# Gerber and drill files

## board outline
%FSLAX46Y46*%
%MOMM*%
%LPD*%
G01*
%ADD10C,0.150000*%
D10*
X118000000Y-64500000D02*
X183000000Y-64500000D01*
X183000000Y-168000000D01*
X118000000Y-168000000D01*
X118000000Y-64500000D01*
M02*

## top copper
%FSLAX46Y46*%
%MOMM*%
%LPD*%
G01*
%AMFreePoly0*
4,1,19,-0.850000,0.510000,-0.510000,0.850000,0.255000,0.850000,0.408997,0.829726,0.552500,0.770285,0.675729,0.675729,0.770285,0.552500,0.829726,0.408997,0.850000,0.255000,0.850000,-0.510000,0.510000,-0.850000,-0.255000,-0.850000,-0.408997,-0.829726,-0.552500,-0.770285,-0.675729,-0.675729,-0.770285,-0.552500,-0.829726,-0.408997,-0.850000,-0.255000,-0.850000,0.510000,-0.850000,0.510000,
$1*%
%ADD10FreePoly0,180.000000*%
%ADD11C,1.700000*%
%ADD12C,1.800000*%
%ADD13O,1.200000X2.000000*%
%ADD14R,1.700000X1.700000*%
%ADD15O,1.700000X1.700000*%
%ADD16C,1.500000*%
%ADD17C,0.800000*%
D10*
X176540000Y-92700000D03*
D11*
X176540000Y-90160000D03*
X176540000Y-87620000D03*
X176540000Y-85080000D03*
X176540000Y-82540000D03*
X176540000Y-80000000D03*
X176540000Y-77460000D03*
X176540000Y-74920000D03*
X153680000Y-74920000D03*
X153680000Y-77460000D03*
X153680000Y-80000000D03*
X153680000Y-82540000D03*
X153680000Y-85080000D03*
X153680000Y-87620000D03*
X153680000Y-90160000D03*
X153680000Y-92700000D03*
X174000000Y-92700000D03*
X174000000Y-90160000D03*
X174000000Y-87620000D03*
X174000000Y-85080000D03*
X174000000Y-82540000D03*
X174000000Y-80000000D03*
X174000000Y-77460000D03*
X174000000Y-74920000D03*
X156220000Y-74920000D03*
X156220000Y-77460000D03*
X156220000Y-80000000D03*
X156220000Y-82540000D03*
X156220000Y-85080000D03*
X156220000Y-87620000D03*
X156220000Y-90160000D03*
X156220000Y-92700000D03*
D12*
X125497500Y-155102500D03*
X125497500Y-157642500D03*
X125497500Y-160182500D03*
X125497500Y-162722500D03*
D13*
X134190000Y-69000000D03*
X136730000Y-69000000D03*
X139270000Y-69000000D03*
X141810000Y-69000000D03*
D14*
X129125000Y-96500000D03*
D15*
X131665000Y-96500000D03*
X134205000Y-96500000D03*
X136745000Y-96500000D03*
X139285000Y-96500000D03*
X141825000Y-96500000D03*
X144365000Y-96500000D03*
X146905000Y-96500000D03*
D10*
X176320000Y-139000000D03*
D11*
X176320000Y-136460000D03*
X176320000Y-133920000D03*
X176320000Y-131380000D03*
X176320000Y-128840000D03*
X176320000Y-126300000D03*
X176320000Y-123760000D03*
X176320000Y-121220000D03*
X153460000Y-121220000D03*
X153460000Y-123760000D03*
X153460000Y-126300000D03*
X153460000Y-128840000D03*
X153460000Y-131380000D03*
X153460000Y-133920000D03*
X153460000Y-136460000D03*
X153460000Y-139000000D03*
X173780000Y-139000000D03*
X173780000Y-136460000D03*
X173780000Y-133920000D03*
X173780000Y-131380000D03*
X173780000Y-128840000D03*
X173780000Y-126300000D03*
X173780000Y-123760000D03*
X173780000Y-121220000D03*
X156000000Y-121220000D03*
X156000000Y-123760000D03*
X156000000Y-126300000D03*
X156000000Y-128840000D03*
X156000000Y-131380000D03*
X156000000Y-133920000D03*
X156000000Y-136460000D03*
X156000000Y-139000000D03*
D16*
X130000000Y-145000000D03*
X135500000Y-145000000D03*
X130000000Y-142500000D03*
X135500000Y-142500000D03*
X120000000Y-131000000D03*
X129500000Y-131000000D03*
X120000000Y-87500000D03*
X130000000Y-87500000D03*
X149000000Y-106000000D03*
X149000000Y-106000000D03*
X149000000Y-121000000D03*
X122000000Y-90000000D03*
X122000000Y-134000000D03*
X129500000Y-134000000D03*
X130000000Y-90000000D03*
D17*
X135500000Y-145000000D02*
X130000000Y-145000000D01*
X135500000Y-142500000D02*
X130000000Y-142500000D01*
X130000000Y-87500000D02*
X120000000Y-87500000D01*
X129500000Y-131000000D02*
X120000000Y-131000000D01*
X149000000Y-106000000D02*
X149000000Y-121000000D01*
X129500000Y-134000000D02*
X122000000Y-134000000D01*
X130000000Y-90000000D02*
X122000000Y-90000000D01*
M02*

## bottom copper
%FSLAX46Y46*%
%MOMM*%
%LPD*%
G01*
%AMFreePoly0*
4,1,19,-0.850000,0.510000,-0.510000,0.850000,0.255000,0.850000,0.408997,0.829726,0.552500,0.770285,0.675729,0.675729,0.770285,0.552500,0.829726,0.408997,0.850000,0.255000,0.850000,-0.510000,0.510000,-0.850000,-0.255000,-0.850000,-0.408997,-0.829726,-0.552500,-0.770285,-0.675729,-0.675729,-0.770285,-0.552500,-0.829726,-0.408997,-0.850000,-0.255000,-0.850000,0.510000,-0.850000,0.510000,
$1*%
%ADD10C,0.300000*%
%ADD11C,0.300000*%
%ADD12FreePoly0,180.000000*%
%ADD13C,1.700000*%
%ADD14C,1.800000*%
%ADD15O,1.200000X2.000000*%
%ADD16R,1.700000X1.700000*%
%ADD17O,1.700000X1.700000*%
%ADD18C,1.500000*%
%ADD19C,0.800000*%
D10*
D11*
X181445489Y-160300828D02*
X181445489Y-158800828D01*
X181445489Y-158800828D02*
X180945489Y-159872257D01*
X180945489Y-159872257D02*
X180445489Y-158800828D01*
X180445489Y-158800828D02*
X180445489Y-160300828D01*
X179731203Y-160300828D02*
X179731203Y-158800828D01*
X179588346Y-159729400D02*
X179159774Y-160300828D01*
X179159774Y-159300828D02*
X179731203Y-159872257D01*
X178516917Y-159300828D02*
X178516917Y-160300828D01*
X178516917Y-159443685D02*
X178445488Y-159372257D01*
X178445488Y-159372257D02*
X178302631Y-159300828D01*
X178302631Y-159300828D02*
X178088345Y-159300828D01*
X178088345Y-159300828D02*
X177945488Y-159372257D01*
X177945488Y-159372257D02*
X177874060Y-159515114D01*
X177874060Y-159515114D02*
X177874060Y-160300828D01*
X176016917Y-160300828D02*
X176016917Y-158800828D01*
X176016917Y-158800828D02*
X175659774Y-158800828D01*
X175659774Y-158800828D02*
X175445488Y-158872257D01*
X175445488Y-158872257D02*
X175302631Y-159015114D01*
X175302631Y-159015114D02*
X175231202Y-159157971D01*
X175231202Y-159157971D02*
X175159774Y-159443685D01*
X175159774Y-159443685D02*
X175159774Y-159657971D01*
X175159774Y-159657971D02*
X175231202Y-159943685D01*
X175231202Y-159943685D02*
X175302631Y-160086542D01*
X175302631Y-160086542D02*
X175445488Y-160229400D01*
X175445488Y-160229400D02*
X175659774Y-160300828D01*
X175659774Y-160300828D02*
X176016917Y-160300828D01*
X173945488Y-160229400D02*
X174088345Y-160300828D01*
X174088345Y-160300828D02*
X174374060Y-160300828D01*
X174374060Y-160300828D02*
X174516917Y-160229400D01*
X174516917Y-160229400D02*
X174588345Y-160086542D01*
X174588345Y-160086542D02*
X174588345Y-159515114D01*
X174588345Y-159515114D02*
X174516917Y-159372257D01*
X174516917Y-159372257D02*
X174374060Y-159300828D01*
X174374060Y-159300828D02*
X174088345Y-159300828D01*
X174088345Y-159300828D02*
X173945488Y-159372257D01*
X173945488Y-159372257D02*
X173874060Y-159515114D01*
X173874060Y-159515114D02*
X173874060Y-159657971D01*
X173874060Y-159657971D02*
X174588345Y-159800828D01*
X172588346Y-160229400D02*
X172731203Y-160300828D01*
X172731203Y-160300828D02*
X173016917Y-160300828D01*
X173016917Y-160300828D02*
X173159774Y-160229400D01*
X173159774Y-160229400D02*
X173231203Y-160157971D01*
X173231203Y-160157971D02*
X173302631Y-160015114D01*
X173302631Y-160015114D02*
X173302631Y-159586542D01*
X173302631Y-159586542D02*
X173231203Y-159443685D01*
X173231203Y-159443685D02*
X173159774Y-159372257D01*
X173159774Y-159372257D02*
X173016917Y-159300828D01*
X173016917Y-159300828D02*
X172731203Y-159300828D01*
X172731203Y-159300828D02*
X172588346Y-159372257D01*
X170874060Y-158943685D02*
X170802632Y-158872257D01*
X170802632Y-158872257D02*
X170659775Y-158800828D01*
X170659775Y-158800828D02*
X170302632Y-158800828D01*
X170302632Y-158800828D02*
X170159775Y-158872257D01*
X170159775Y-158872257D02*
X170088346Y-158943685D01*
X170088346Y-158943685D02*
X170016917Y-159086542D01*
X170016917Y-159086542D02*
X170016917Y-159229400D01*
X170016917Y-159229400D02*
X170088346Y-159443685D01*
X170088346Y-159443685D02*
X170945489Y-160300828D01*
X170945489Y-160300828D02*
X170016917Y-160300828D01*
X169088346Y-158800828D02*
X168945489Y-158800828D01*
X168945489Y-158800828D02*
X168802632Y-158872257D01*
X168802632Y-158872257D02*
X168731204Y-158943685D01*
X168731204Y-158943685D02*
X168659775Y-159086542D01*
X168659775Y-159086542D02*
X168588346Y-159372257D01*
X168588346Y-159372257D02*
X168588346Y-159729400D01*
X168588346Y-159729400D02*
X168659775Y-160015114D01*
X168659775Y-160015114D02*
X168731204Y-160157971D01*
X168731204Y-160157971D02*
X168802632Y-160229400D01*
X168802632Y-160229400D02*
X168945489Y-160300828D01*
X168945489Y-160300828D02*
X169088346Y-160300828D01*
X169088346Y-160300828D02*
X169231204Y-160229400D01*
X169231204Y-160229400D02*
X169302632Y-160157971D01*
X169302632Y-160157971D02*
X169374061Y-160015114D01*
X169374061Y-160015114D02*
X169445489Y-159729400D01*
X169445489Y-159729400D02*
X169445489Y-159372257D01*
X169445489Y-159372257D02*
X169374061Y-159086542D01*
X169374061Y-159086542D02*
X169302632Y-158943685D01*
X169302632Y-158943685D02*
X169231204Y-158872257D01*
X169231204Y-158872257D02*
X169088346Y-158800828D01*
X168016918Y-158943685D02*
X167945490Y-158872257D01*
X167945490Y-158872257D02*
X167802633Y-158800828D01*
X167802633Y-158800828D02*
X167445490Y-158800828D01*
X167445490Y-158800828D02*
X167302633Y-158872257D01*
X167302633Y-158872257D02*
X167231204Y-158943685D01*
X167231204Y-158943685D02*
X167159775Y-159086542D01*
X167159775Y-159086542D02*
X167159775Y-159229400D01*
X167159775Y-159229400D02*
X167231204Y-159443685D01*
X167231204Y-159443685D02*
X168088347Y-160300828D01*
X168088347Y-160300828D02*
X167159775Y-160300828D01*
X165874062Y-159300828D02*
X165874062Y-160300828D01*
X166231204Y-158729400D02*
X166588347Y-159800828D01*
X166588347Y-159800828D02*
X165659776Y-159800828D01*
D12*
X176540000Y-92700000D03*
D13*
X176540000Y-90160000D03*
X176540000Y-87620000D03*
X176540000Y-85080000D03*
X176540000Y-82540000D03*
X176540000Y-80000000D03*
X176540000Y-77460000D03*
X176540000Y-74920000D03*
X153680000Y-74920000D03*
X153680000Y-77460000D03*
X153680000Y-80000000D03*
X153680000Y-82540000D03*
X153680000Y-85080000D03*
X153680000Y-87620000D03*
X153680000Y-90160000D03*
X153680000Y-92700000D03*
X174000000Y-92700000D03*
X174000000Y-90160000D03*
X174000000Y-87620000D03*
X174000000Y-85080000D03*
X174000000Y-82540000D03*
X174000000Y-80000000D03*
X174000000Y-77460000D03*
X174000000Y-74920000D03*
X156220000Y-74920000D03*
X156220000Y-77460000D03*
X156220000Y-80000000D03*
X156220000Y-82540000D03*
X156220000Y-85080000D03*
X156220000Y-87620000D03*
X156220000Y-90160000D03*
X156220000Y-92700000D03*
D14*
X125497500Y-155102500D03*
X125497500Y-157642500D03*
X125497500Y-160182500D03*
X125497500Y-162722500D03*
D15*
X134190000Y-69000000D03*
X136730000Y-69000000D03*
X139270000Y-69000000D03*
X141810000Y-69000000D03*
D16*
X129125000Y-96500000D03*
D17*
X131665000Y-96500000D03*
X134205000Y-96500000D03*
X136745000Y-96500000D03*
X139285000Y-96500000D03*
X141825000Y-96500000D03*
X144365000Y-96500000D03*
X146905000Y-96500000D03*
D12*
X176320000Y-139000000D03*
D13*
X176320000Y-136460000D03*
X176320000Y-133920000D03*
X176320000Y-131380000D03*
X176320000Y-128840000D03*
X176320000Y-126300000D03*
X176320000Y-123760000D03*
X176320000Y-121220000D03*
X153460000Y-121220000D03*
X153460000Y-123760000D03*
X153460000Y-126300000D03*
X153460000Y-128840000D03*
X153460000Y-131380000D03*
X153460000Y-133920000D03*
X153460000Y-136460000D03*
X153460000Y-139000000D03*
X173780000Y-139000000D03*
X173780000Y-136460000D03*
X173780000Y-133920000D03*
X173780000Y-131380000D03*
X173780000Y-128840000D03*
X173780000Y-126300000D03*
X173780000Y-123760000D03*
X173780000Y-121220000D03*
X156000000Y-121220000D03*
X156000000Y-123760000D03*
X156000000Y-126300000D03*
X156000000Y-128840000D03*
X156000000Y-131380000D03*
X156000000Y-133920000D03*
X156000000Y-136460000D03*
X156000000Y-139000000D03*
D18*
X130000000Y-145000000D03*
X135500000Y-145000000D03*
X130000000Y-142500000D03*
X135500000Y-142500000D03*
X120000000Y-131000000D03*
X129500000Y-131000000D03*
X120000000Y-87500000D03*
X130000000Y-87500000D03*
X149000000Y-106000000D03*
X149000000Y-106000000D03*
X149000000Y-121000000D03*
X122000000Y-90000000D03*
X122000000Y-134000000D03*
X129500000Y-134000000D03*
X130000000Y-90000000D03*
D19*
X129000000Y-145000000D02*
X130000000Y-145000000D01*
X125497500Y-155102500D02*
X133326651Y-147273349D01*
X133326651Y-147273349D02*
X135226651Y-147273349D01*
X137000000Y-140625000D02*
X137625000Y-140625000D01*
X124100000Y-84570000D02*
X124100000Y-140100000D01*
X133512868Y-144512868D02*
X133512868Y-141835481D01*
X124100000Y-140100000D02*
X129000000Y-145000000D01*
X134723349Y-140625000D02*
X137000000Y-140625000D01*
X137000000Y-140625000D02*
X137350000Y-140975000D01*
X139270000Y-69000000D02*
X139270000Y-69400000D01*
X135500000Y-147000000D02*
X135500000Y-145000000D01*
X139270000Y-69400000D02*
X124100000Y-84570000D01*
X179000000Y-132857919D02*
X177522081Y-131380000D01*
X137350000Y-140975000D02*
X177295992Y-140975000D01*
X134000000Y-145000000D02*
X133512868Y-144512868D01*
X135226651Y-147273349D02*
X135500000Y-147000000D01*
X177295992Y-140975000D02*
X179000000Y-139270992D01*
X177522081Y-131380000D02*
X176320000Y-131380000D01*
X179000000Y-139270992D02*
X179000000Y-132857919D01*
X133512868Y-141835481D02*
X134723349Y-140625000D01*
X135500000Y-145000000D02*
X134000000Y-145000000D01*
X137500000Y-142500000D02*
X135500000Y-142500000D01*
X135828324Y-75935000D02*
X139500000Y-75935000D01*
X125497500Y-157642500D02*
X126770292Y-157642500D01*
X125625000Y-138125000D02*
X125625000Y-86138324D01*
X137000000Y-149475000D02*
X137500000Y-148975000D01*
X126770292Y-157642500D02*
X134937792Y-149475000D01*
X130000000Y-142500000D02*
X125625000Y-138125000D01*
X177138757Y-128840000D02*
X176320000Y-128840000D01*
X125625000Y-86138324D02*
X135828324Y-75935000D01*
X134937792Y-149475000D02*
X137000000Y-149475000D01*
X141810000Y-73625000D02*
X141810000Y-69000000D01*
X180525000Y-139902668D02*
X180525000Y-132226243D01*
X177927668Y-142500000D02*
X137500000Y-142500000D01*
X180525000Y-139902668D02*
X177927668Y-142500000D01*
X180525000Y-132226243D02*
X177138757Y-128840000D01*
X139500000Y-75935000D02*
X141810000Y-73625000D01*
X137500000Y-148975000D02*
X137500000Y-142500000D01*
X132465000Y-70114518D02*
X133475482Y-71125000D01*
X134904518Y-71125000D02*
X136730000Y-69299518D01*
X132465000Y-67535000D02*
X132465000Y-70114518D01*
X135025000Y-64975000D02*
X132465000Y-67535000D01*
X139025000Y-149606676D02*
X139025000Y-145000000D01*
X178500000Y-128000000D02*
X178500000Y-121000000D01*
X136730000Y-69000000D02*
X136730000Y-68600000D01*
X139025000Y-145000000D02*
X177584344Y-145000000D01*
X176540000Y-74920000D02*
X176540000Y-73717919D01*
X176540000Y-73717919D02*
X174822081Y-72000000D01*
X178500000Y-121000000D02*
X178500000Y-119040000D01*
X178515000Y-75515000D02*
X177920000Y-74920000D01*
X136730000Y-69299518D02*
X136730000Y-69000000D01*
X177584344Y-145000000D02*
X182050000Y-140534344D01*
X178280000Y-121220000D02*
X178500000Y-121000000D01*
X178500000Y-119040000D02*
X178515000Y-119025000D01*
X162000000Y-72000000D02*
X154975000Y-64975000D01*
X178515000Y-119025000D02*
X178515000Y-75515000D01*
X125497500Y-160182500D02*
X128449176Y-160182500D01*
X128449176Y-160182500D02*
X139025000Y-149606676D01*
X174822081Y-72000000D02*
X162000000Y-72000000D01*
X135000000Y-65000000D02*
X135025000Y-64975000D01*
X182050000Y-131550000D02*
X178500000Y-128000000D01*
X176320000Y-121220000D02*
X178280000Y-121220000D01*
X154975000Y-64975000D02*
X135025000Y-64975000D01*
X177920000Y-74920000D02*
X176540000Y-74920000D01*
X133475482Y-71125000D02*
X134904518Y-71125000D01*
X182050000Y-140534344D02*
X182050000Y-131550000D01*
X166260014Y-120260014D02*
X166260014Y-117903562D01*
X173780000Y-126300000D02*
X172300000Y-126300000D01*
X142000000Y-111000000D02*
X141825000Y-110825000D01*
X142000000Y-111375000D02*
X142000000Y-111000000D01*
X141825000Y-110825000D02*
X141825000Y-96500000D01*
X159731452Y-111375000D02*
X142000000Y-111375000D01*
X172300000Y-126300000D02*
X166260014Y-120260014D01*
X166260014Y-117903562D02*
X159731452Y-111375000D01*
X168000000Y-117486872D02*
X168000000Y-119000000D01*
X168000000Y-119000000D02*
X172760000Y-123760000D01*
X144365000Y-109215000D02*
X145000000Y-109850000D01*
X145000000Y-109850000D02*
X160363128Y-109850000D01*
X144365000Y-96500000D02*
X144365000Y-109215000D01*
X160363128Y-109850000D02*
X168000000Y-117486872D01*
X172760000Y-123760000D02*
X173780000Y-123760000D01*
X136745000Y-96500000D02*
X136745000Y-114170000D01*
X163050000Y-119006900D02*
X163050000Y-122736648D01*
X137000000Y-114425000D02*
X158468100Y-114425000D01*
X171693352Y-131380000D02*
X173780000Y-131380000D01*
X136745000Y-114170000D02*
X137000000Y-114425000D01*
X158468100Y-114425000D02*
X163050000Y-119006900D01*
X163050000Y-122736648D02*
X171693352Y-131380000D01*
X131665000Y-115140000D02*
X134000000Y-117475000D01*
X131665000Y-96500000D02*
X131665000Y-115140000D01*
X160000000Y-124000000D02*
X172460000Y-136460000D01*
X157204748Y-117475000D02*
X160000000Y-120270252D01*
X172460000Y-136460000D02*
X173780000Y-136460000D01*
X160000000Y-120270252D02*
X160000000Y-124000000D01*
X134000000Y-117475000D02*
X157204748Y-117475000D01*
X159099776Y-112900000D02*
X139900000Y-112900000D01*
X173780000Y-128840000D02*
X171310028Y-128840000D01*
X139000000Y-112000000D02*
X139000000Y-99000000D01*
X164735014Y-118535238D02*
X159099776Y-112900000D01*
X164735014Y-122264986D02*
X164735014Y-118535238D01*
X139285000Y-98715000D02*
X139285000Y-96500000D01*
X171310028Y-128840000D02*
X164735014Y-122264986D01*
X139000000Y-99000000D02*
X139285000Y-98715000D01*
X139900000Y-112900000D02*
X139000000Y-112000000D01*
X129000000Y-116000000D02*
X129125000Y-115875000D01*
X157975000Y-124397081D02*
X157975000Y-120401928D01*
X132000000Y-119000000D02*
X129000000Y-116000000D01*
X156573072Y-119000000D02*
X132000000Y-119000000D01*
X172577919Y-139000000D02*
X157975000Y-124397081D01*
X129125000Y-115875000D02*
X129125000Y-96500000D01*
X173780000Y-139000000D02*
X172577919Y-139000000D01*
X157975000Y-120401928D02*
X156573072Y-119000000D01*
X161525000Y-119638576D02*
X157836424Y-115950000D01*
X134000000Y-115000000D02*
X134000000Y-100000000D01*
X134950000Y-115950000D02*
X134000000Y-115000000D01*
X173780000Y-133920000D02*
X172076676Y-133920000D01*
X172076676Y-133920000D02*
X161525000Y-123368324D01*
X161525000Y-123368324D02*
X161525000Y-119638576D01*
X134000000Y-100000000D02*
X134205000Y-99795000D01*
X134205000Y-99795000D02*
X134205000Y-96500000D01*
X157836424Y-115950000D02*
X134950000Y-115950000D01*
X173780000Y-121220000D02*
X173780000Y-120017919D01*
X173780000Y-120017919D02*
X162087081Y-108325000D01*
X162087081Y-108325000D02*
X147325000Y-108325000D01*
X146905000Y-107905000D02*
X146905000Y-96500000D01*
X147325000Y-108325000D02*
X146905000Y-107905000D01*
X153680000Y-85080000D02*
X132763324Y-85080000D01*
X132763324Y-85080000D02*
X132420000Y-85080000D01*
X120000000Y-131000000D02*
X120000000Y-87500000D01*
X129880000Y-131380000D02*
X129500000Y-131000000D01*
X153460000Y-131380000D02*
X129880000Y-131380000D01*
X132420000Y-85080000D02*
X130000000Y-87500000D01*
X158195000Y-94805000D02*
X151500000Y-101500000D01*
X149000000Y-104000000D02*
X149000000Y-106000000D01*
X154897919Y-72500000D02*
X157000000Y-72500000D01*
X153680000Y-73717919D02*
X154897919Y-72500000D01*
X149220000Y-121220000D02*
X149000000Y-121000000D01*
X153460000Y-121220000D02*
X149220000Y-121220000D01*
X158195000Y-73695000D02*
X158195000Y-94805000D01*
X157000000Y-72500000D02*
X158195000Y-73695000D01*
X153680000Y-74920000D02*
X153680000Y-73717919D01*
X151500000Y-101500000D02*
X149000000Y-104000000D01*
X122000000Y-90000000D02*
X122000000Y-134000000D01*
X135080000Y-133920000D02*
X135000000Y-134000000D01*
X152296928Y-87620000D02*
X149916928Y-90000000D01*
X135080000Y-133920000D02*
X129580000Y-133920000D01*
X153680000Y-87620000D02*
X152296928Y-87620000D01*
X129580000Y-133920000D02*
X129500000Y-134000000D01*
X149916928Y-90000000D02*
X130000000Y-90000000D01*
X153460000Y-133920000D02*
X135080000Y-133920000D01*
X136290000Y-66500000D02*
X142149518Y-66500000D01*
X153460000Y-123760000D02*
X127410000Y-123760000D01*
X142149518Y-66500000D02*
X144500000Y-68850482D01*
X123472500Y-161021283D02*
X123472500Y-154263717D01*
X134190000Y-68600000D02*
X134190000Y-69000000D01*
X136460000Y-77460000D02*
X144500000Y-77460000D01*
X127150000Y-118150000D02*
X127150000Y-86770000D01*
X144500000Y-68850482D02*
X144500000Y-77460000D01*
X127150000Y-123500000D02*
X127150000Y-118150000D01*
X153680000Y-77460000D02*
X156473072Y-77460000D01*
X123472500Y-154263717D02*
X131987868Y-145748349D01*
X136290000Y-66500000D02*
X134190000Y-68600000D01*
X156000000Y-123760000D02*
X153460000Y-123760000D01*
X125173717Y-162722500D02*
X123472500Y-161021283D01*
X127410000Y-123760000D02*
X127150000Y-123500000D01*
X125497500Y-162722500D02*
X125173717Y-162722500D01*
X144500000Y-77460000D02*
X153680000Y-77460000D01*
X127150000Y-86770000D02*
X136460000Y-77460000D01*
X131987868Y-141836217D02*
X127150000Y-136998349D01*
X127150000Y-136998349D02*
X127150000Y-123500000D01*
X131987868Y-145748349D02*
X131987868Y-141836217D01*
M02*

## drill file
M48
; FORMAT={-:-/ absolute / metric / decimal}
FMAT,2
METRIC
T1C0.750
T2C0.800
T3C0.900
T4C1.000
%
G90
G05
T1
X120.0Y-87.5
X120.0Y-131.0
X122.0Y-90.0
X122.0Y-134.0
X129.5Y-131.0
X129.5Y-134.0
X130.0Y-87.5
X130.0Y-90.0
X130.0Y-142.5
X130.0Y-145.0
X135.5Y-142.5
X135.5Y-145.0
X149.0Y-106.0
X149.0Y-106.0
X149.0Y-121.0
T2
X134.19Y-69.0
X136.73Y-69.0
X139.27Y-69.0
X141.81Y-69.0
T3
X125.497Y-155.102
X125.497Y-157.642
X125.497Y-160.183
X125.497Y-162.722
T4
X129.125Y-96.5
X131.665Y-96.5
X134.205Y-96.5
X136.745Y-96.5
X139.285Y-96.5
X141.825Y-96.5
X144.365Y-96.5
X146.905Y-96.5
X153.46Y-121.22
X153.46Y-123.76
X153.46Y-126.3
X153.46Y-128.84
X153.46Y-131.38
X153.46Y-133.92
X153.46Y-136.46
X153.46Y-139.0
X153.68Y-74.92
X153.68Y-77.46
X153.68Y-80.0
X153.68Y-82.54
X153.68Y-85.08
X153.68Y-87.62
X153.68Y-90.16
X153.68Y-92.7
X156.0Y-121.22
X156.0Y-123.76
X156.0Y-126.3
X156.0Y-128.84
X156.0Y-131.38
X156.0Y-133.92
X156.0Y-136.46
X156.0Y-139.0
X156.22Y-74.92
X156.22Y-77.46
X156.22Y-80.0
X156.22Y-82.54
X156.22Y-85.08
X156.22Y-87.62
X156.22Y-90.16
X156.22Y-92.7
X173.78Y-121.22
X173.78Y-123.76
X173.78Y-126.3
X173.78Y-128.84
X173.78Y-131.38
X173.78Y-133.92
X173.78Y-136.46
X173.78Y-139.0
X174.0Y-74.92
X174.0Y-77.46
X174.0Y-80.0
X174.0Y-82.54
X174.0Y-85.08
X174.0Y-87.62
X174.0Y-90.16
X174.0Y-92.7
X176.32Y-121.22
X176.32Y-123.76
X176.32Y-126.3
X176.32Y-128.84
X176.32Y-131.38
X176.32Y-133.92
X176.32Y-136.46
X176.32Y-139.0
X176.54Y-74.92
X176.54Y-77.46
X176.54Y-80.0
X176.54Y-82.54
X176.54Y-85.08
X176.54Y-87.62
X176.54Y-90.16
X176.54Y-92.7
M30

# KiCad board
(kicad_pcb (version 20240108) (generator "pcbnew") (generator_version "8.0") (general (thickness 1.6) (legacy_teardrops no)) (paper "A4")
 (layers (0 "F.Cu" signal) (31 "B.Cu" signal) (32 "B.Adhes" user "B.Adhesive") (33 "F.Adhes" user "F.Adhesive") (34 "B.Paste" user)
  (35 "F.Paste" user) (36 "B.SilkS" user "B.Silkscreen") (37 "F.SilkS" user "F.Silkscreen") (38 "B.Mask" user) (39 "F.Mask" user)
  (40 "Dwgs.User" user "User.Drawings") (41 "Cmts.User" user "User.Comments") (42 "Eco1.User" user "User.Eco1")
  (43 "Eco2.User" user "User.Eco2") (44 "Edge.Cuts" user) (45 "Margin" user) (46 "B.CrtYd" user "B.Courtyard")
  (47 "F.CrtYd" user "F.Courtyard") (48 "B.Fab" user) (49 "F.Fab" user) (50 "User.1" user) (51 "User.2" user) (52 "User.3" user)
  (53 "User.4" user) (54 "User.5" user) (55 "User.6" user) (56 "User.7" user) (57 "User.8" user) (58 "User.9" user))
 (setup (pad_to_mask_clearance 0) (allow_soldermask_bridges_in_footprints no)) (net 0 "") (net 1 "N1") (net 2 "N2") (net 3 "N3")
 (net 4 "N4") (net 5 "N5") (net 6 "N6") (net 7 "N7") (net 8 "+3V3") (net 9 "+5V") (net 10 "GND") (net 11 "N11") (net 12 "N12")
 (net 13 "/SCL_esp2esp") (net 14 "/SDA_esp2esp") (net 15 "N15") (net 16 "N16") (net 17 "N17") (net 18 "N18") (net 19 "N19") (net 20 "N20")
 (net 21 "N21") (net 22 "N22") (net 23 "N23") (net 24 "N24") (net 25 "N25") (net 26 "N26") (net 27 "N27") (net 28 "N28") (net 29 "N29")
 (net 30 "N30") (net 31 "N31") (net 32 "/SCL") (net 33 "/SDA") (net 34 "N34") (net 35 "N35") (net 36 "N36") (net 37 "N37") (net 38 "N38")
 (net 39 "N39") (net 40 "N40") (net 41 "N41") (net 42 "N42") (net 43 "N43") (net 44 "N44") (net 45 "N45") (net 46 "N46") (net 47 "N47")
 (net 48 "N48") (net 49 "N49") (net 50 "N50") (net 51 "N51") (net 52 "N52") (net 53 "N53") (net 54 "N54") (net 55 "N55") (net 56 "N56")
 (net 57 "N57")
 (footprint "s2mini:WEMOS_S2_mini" (layer "F.Cu") (at 176.54 92.7 180)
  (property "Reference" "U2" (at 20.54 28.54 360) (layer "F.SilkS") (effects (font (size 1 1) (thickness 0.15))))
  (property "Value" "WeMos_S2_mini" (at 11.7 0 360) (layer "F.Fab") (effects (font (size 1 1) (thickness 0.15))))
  (pad "1" thru_hole roundrect (at 0 0 180) (size 1.7 1.7) (drill 1) (layers "*.Cu" "*.Mask") (remove_unused_layers no)
   (roundrect_rratio 0.35) (chamfer_ratio 0.2) (chamfer top_left bottom_right) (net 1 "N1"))
  (pad "2" thru_hole circle (at 0 2.54 180) (size 1.7 1.7) (drill 1) (layers "*.Cu" "*.Mask") (remove_unused_layers no) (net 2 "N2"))
  (pad "3" thru_hole circle (at 0 5.08 180) (size 1.7 1.7) (drill 1) (layers "*.Cu" "*.Mask") (remove_unused_layers no) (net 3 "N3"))
  (pad "4" thru_hole circle (at 0 7.62 180) (size 1.7 1.7) (drill 1) (layers "*.Cu" "*.Mask") (remove_unused_layers no) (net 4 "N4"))
  (pad "5" thru_hole circle (at 0 10.16 180) (size 1.7 1.7) (drill 1) (layers "*.Cu" "*.Mask") (remove_unused_layers no) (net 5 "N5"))
  (pad "6" thru_hole circle (at 0 12.7 180) (size 1.7 1.7) (drill 1) (layers "*.Cu" "*.Mask") (remove_unused_layers no) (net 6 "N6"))
  (pad "7" thru_hole circle (at 0 15.24 180) (size 1.7 1.7) (drill 1) (layers "*.Cu" "*.Mask") (remove_unused_layers no) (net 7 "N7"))
  (pad "8" thru_hole circle (at 0 17.78 180) (size 1.7 1.7) (drill 1) (layers "*.Cu" "*.Mask") (remove_unused_layers no) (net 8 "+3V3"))
  (pad "9" thru_hole circle (at 22.86 17.78 180) (size 1.7 1.7) (drill 1) (layers "*.Cu" "*.Mask") (remove_unused_layers no) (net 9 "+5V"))
  (pad "10" thru_hole circle (at 22.86 15.24 180) (size 1.7 1.7) (drill 1) (layers "*.Cu" "*.Mask") (remove_unused_layers no) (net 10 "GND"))
  (pad "11" thru_hole circle (at 22.86 12.7 180) (size 1.7 1.7) (drill 1) (layers "*.Cu" "*.Mask") (remove_unused_layers no) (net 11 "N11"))
  (pad "12" thru_hole circle (at 22.86 10.16 180) (size 1.7 1.7) (drill 1) (layers "*.Cu" "*.Mask") (remove_unused_layers no) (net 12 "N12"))
  (pad "13" thru_hole circle (at 22.86 7.62 180) (size 1.7 1.7) (drill 1) (layers "*.Cu" "*.Mask") (remove_unused_layers no)
   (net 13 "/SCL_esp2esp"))
  (pad "14" thru_hole circle (at 22.86 5.08 180) (size 1.7 1.7) (drill 1) (layers "*.Cu" "*.Mask") (remove_unused_layers no)
   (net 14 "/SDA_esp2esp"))
  (pad "15" thru_hole circle (at 22.86 2.54 180) (size 1.7 1.7) (drill 1) (layers "*.Cu" "*.Mask") (remove_unused_layers no) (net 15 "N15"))
  (pad "16" thru_hole circle (at 22.86 0 180) (size 1.7 1.7) (drill 1) (layers "*.Cu" "*.Mask") (remove_unused_layers no) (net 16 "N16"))
  (pad "17" thru_hole circle (at 2.54 0 180) (size 1.7 1.7) (drill 1) (layers "*.Cu" "*.Mask") (remove_unused_layers no) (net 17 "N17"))
  (pad "18" thru_hole circle (at 2.54 2.54 180) (size 1.7 1.7) (drill 1) (layers "*.Cu" "*.Mask") (remove_unused_layers no) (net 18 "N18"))
  (pad "19" thru_hole circle (at 2.54 5.08 180) (size 1.7 1.7) (drill 1) (layers "*.Cu" "*.Mask") (remove_unused_layers no) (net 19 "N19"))
  (pad "20" thru_hole circle (at 2.54 7.62 180) (size 1.7 1.7) (drill 1) (layers "*.Cu" "*.Mask") (remove_unused_layers no) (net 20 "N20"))
  (pad "21" thru_hole circle (at 2.54 10.16 180) (size 1.7 1.7) (drill 1) (layers "*.Cu" "*.Mask") (remove_unused_layers no) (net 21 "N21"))
  (pad "22" thru_hole circle (at 2.54 12.7 180) (size 1.7 1.7) (drill 1) (layers "*.Cu" "*.Mask") (remove_unused_layers no) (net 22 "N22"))
  (pad "23" thru_hole circle (at 2.54 15.24 180) (size 1.7 1.7) (drill 1) (layers "*.Cu" "*.Mask") (remove_unused_layers no) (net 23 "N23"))
  (pad "24" thru_hole circle (at 2.54 17.78 180) (size 1.7 1.7) (drill 1) (layers "*.Cu" "*.Mask") (remove_unused_layers no) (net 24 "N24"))
  (pad "25" thru_hole circle (at 20.32 17.78 180) (size 1.7 1.7) (drill 1) (layers "*.Cu" "*.Mask") (remove_unused_layers no) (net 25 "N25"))
  (pad "26" thru_hole circle (at 20.32 15.24 180) (size 1.7 1.7) (drill 1) (layers "*.Cu" "*.Mask") (remove_unused_layers no) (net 10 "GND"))
  (pad "27" thru_hole circle (at 20.32 12.7 180) (size 1.7 1.7) (drill 1) (layers "*.Cu" "*.Mask") (remove_unused_layers no) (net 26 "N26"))
  (pad "28" thru_hole circle (at 20.32 10.16 180) (size 1.7 1.7) (drill 1) (layers "*.Cu" "*.Mask") (remove_unused_layers no) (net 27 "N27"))
  (pad "29" thru_hole circle (at 20.32 7.62 180) (size 1.7 1.7) (drill 1) (layers "*.Cu" "*.Mask") (remove_unused_layers no) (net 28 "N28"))
  (pad "30" thru_hole circle (at 20.32 5.08 180) (size 1.7 1.7) (drill 1) (layers "*.Cu" "*.Mask") (remove_unused_layers no) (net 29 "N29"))
  (pad "31" thru_hole circle (at 20.32 2.54 180) (size 1.7 1.7) (drill 1) (layers "*.Cu" "*.Mask") (remove_unused_layers no) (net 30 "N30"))
  (pad "32" thru_hole circle (at 20.32 0 180) (size 1.7 1.7) (drill 1) (layers "*.Cu" "*.Mask") (remove_unused_layers no) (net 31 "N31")))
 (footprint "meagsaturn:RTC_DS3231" (layer "F.Cu") (at 163.5975 170.3425 180)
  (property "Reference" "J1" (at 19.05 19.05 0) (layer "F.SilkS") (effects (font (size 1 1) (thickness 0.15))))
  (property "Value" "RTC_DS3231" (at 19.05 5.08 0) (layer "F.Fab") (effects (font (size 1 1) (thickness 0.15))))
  (pad "1" thru_hole circle (at 38.1 15.24 180) (size 1.8 1.8) (drill 0.9) (layers "*.Cu" "*.Mask") (remove_unused_layers no)
   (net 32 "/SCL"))
  (pad "2" thru_hole circle (at 38.1 12.7 180) (size 1.8 1.8) (drill 0.9) (layers "*.Cu" "*.Mask") (remove_unused_layers no) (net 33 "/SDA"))
  (pad "3" thru_hole circle (at 38.1 10.16 180) (size 1.8 1.8) (drill 0.9) (layers "*.Cu" "*.Mask") (remove_unused_layers no) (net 8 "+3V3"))
  (pad "4" thru_hole circle (at 38.1 7.62 180) (size 1.8 1.8) (drill 0.9) (layers "*.Cu" "*.Mask") (remove_unused_layers no) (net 10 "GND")))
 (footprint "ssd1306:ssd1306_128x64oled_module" (layer "F.Cu") (at 138 69)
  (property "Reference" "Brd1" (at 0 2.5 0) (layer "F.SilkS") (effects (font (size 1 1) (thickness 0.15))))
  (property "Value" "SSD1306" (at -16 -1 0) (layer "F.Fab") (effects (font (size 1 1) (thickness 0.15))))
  (pad "1" thru_hole oval (at -3.81 0) (size 1.2 2) (drill 0.8) (layers "*.Cu" "*.Mask") (remove_unused_layers no) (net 10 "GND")
   (thermal_bridge_angle 45))
  (pad "2" thru_hole oval (at -1.27 0) (size 1.2 2) (drill 0.8) (layers "*.Cu" "*.Mask") (remove_unused_layers no) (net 8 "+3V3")
   (thermal_bridge_angle 45))
  (pad "3" thru_hole oval (at 1.27 0) (size 1.2 2) (drill 0.8) (layers "*.Cu" "*.Mask") (remove_unused_layers no) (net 32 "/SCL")
   (thermal_bridge_angle 45))
  (pad "4" thru_hole oval (at 3.81 0) (size 1.2 2) (drill 0.8) (layers "*.Cu" "*.Mask") (remove_unused_layers no) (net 33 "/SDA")
   (thermal_bridge_angle 45)))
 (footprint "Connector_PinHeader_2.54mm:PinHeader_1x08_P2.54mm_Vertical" (layer "F.Cu") (at 129.125 96.5 90)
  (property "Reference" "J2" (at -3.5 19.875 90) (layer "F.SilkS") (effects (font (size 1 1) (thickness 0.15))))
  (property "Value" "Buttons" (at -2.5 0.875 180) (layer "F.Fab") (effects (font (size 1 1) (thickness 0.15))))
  (pad "1" thru_hole rect (at 0 0 90) (size 1.7 1.7) (drill 1) (layers "*.Cu" "*.Mask") (remove_unused_layers no) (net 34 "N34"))
  (pad "2" thru_hole oval (at 0 2.54 90) (size 1.7 1.7) (drill 1) (layers "*.Cu" "*.Mask") (remove_unused_layers no) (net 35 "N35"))
  (pad "3" thru_hole oval (at 0 5.08 90) (size 1.7 1.7) (drill 1) (layers "*.Cu" "*.Mask") (remove_unused_layers no) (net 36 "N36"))
  (pad "4" thru_hole oval (at 0 7.62 90) (size 1.7 1.7) (drill 1) (layers "*.Cu" "*.Mask") (remove_unused_layers no) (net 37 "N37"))
  (pad "5" thru_hole oval (at 0 10.16 90) (size 1.7 1.7) (drill 1) (layers "*.Cu" "*.Mask") (remove_unused_layers no) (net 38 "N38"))
  (pad "6" thru_hole oval (at 0 12.7 90) (size 1.7 1.7) (drill 1) (layers "*.Cu" "*.Mask") (remove_unused_layers no) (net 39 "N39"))
  (pad "7" thru_hole oval (at 0 15.24 90) (size 1.7 1.7) (drill 1) (layers "*.Cu" "*.Mask") (remove_unused_layers no) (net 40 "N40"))
  (pad "8" thru_hole oval (at 0 17.78 90) (size 1.7 1.7) (drill 1) (layers "*.Cu" "*.Mask") (remove_unused_layers no) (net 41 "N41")))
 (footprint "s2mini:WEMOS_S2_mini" (layer "F.Cu") (at 176.32 139 180)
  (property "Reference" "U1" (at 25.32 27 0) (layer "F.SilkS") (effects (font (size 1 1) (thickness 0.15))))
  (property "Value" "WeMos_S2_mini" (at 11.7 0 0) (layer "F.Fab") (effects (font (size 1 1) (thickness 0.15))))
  (pad "1" thru_hole roundrect (at 0 0 180) (size 1.7 1.7) (drill 1) (layers "*.Cu" "*.Mask") (remove_unused_layers no)
   (roundrect_rratio 0.35) (chamfer_ratio 0.2) (chamfer top_left bottom_right) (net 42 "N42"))
  (pad "2" thru_hole circle (at 0 2.54 180) (size 1.7 1.7) (drill 1) (layers "*.Cu" "*.Mask") (remove_unused_layers no) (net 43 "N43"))
  (pad "3" thru_hole circle (at 0 5.08 180) (size 1.7 1.7) (drill 1) (layers "*.Cu" "*.Mask") (remove_unused_layers no) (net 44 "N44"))
  (pad "4" thru_hole circle (at 0 7.62 180) (size 1.7 1.7) (drill 1) (layers "*.Cu" "*.Mask") (remove_unused_layers no) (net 32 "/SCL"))
  (pad "5" thru_hole circle (at 0 10.16 180) (size 1.7 1.7) (drill 1) (layers "*.Cu" "*.Mask") (remove_unused_layers no) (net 33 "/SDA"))
  (pad "6" thru_hole circle (at 0 12.7 180) (size 1.7 1.7) (drill 1) (layers "*.Cu" "*.Mask") (remove_unused_layers no) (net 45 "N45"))
  (pad "7" thru_hole circle (at 0 15.24 180) (size 1.7 1.7) (drill 1) (layers "*.Cu" "*.Mask") (remove_unused_layers no) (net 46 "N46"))
  (pad "8" thru_hole circle (at 0 17.78 180) (size 1.7 1.7) (drill 1) (layers "*.Cu" "*.Mask") (remove_unused_layers no) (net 8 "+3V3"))
  (pad "9" thru_hole circle (at 22.86 17.78 180) (size 1.7 1.7) (drill 1) (layers "*.Cu" "*.Mask") (remove_unused_layers no) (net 9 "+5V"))
  (pad "10" thru_hole circle (at 22.86 15.24 180) (size 1.7 1.7) (drill 1) (layers "*.Cu" "*.Mask") (remove_unused_layers no) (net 10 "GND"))
  (pad "11" thru_hole circle (at 22.86 12.7 180) (size 1.7 1.7) (drill 1) (layers "*.Cu" "*.Mask") (remove_unused_layers no) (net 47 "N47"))
  (pad "12" thru_hole circle (at 22.86 10.16 180) (size 1.7 1.7) (drill 1) (layers "*.Cu" "*.Mask") (remove_unused_layers no) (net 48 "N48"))
  (pad "13" thru_hole circle (at 22.86 7.62 180) (size 1.7 1.7) (drill 1) (layers "*.Cu" "*.Mask") (remove_unused_layers no)
   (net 13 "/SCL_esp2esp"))
  (pad "14" thru_hole circle (at 22.86 5.08 180) (size 1.7 1.7) (drill 1) (layers "*.Cu" "*.Mask") (remove_unused_layers no)
   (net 14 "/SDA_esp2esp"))
  (pad "15" thru_hole circle (at 22.86 2.54 180) (size 1.7 1.7) (drill 1) (layers "*.Cu" "*.Mask") (remove_unused_layers no) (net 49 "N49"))
  (pad "16" thru_hole circle (at 22.86 0 180) (size 1.7 1.7) (drill 1) (layers "*.Cu" "*.Mask") (remove_unused_layers no) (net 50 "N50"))
  (pad "17" thru_hole circle (at 2.54 0 180) (size 1.7 1.7) (drill 1) (layers "*.Cu" "*.Mask") (remove_unused_layers no) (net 34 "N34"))
  (pad "18" thru_hole circle (at 2.54 2.54 180) (size 1.7 1.7) (drill 1) (layers "*.Cu" "*.Mask") (remove_unused_layers no) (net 35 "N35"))
  (pad "19" thru_hole circle (at 2.54 5.08 180) (size 1.7 1.7) (drill 1) (layers "*.Cu" "*.Mask") (remove_unused_layers no) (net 36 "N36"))
  (pad "20" thru_hole circle (at 2.54 7.62 180) (size 1.7 1.7) (drill 1) (layers "*.Cu" "*.Mask") (remove_unused_layers no) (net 37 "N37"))
  (pad "21" thru_hole circle (at 2.54 10.16 180) (size 1.7 1.7) (drill 1) (layers "*.Cu" "*.Mask") (remove_unused_layers no) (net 38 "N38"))
  (pad "22" thru_hole circle (at 2.54 12.7 180) (size 1.7 1.7) (drill 1) (layers "*.Cu" "*.Mask") (remove_unused_layers no) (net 39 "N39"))
  (pad "23" thru_hole circle (at 2.54 15.24 180) (size 1.7 1.7) (drill 1) (layers "*.Cu" "*.Mask") (remove_unused_layers no) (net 40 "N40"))
  (pad "24" thru_hole circle (at 2.54 17.78 180) (size 1.7 1.7) (drill 1) (layers "*.Cu" "*.Mask") (remove_unused_layers no) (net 41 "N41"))
  (pad "25" thru_hole circle (at 20.32 17.78 180) (size 1.7 1.7) (drill 1) (layers "*.Cu" "*.Mask") (remove_unused_layers no) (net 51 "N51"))
  (pad "26" thru_hole circle (at 20.32 15.24 180) (size 1.7 1.7) (drill 1) (layers "*.Cu" "*.Mask") (remove_unused_layers no) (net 10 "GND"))
  (pad "27" thru_hole circle (at 20.32 12.7 180) (size 1.7 1.7) (drill 1) (layers "*.Cu" "*.Mask") (remove_unused_layers no) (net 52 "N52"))
  (pad "28" thru_hole circle (at 20.32 10.16 180) (size 1.7 1.7) (drill 1) (layers "*.Cu" "*.Mask") (remove_unused_layers no) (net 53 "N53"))
  (pad "29" thru_hole circle (at 20.32 7.62 180) (size 1.7 1.7) (drill 1) (layers "*.Cu" "*.Mask") (remove_unused_layers no) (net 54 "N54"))
  (pad "30" thru_hole circle (at 20.32 5.08 180) (size 1.7 1.7) (drill 1) (layers "*.Cu" "*.Mask") (remove_unused_layers no) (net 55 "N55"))
  (pad "31" thru_hole circle (at 20.32 2.54 180) (size 1.7 1.7) (drill 1) (layers "*.Cu" "*.Mask") (remove_unused_layers no) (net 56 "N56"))
  (pad "32" thru_hole circle (at 20.32 0 180) (size 1.7 1.7) (drill 1) (layers "*.Cu" "*.Mask") (remove_unused_layers no) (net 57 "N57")))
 (gr_rect (start 118 64.5) (end 183 168) (stroke (width 0.15) (type default)) (fill none) (layer "Edge.Cuts"))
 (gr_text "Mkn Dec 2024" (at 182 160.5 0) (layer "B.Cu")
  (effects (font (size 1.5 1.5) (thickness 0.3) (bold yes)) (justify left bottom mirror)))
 (segment (start 135.5 145) (end 130 145) (width 0.8) (layer "F.Cu") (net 32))
 (via (at 130 145) (size 1.5) (drill 0.75) (layers "F.Cu" "B.Cu") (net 32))
 (via (at 135.5 145) (size 1.5) (drill 0.75) (layers "F.Cu" "B.Cu") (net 32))
 (segment (start 129 145) (end 130 145) (width 0.8) (layer "B.Cu") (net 32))
 (segment (start 125.4975 155.1025) (end 133.326651 147.273349) (width 0.8) (layer "B.Cu") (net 32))
 (segment (start 133.326651 147.273349) (end 135.226651 147.273349) (width 0.8) (layer "B.Cu") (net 32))
 (segment (start 137 140.625) (end 137.625 140.625) (width 0.8) (layer "B.Cu") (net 32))
 (segment (start 124.1 84.57) (end 124.1 140.1) (width 0.8) (layer "B.Cu") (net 32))
 (segment (start 133.512868 144.512868) (end 133.512868 141.835481) (width 0.8) (layer "B.Cu") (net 32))
 (segment (start 124.1 140.1) (end 129 145) (width 0.8) (layer "B.Cu") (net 32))
 (segment (start 134.723349 140.625) (end 137 140.625) (width 0.8) (layer "B.Cu") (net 32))
 (segment (start 137 140.625) (end 137.35 140.975) (width 0.8) (layer "B.Cu") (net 32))
 (segment (start 139.27 69) (end 139.27 69.4) (width 0.8) (layer "B.Cu") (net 32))
 (segment (start 135.5 147) (end 135.5 145) (width 0.8) (layer "B.Cu") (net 32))
 (segment (start 139.27 69.4) (end 124.1 84.57) (width 0.8) (layer "B.Cu") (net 32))
 (segment (start 179 132.857919) (end 177.522081 131.38) (width 0.8) (layer "B.Cu") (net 32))
 (segment (start 137.35 140.975) (end 177.295992 140.975) (width 0.8) (layer "B.Cu") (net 32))
 (segment (start 134 145) (end 133.512868 144.512868) (width 0.8) (layer "B.Cu") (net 32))
 (segment (start 135.226651 147.273349) (end 135.5 147) (width 0.8) (layer "B.Cu") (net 32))
 (segment (start 177.295992 140.975) (end 179 139.270992) (width 0.8) (layer "B.Cu") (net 32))
 (segment (start 177.522081 131.38) (end 176.32 131.38) (width 0.8) (layer "B.Cu") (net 32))
 (segment (start 179 139.270992) (end 179 132.857919) (width 0.8) (layer "B.Cu") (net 32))
 (segment (start 133.512868 141.835481) (end 134.723349 140.625) (width 0.8) (layer "B.Cu") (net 32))
 (segment (start 135.5 145) (end 134 145) (width 0.8) (layer "B.Cu") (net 32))
 (segment (start 135.5 142.5) (end 130 142.5) (width 0.8) (layer "F.Cu") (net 33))
 (via (at 130 142.5) (size 1.5) (drill 0.75) (layers "F.Cu" "B.Cu") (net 33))
 (via (at 135.5 142.5) (size 1.5) (drill 0.75) (layers "F.Cu" "B.Cu") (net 33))
 (segment (start 137.5 142.5) (end 135.5 142.5) (width 0.8) (layer "B.Cu") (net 33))
 (segment (start 135.828324 75.935) (end 139.5 75.935) (width 0.8) (layer "B.Cu") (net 33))
 (segment (start 125.4975 157.6425) (end 126.770292 157.6425) (width 0.8) (layer "B.Cu") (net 33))
 (segment (start 125.625 138.125) (end 125.625 86.138324) (width 0.8) (layer "B.Cu") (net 33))
 (segment (start 137 149.475) (end 137.5 148.975) (width 0.8) (layer "B.Cu") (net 33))
 (segment (start 126.770292 157.6425) (end 134.937792 149.475) (width 0.8) (layer "B.Cu") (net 33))
 (segment (start 130 142.5) (end 125.625 138.125) (width 0.8) (layer "B.Cu") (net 33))
 (segment (start 177.138757 128.84) (end 176.32 128.84) (width 0.8) (layer "B.Cu") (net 33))
 (segment (start 125.625 86.138324) (end 135.828324 75.935) (width 0.8) (layer "B.Cu") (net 33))
 (segment (start 134.937792 149.475) (end 137 149.475) (width 0.8) (layer "B.Cu") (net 33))
 (segment (start 141.81 73.625) (end 141.81 69) (width 0.8) (layer "B.Cu") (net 33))
 (segment (start 180.525 139.902668) (end 180.525 132.226243) (width 0.8) (layer "B.Cu") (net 33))
 (segment (start 177.927668 142.5) (end 137.5 142.5) (width 0.8) (layer "B.Cu") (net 33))
 (segment (start 180.525 139.902668) (end 177.927668 142.5) (width 0.8) (layer "B.Cu") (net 33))
 (segment (start 180.525 132.226243) (end 177.138757 128.84) (width 0.8) (layer "B.Cu") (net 33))
 (segment (start 139.5 75.935) (end 141.81 73.625) (width 0.8) (layer "B.Cu") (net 33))
 (segment (start 137.5 148.975) (end 137.5 142.5) (width 0.8) (layer "B.Cu") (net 33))
 (segment (start 132.465 70.114518) (end 133.475482 71.125) (width 0.8) (layer "B.Cu") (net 8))
 (segment (start 134.904518 71.125) (end 136.73 69.299518) (width 0.8) (layer "B.Cu") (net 8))
 (segment (start 132.465 67.535) (end 132.465 70.114518) (width 0.8) (layer "B.Cu") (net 8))
 (segment (start 135.025 64.975) (end 132.465 67.535) (width 0.8) (layer "B.Cu") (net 8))
 (segment (start 139.025 149.606676) (end 139.025 145) (width 0.8) (layer "B.Cu") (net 8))
 (segment (start 178.5 128) (end 178.5 121) (width 0.8) (layer "B.Cu") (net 8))
 (segment (start 136.73 69) (end 136.73 68.6) (width 0.8) (layer "B.Cu") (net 8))
 (segment (start 139.025 145) (end 177.584344 145) (width 0.8) (layer "B.Cu") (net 8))
 (segment (start 176.54 74.92) (end 176.54 73.717919) (width 0.8) (layer "B.Cu") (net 8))
 (segment (start 176.54 73.717919) (end 174.822081 72) (width 0.8) (layer "B.Cu") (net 8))
 (segment (start 178.5 121) (end 178.5 119.04) (width 0.8) (layer "B.Cu") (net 8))
 (segment (start 178.515 75.515) (end 177.92 74.92) (width 0.8) (layer "B.Cu") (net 8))
 (segment (start 136.73 69.299518) (end 136.73 69) (width 0.8) (layer "B.Cu") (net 8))
 (segment (start 177.584344 145) (end 182.05 140.534344) (width 0.8) (layer "B.Cu") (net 8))
 (segment (start 178.28 121.22) (end 178.5 121) (width 0.8) (layer "B.Cu") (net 8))
 (segment (start 178.5 119.04) (end 178.515 119.025) (width 0.8) (layer "B.Cu") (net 8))
 (segment (start 162 72) (end 154.975 64.975) (width 0.8) (layer "B.Cu") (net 8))
 (segment (start 178.515 119.025) (end 178.515 75.515) (width 0.8) (layer "B.Cu") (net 8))
 (segment (start 125.4975 160.1825) (end 128.449176 160.1825) (width 0.8) (layer "B.Cu") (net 8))
 (segment (start 128.449176 160.1825) (end 139.025 149.606676) (width 0.8) (layer "B.Cu") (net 8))
 (segment (start 174.822081 72) (end 162 72) (width 0.8) (layer "B.Cu") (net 8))
 (segment (start 135 65) (end 135.025 64.975) (width 0.8) (layer "B.Cu") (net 8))
 (segment (start 182.05 131.55) (end 178.5 128) (width 0.8) (layer "B.Cu") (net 8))
 (segment (start 176.32 121.22) (end 178.28 121.22) (width 0.8) (layer "B.Cu") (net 8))
 (segment (start 154.975 64.975) (end 135.025 64.975) (width 0.8) (layer "B.Cu") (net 8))
 (segment (start 177.92 74.92) (end 176.54 74.92) (width 0.8) (layer "B.Cu") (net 8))
 (segment (start 133.475482 71.125) (end 134.904518 71.125) (width 0.8) (layer "B.Cu") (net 8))
 (segment (start 182.05 140.534344) (end 182.05 131.55) (width 0.8) (layer "B.Cu") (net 8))
 (segment (start 166.260014 120.260014) (end 166.260014 117.903562) (width 0.8) (layer "B.Cu") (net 39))
 (segment (start 173.78 126.3) (end 172.3 126.3) (width 0.8) (layer "B.Cu") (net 39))
 (segment (start 142 111) (end 141.825 110.825) (width 0.8) (layer "B.Cu") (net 39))
 (segment (start 142 111.375) (end 142 111) (width 0.8) (layer "B.Cu") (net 39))
 (segment (start 141.825 110.825) (end 141.825 96.5) (width 0.8) (layer "B.Cu") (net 39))
 (segment (start 159.731452 111.375) (end 142 111.375) (width 0.8) (layer "B.Cu") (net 39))
 (segment (start 172.3 126.3) (end 166.260014 120.260014) (width 0.8) (layer "B.Cu") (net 39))
 (segment (start 166.260014 117.903562) (end 159.731452 111.375) (width 0.8) (layer "B.Cu") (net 39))
 (segment (start 168 117.486872) (end 168 119) (width 0.8) (layer "B.Cu") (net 40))
 (segment (start 168 119) (end 172.76 123.76) (width 0.8) (layer "B.Cu") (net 40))
 (segment (start 144.365 109.215) (end 145 109.85) (width 0.8) (layer "B.Cu") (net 40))
 (segment (start 145 109.85) (end 160.363128 109.85) (width 0.8) (layer "B.Cu") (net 40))
 (segment (start 144.365 96.5) (end 144.365 109.215) (width 0.8) (layer "B.Cu") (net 40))
 (segment (start 160.363128 109.85) (end 168 117.486872) (width 0.8) (layer "B.Cu") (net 40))
 (segment (start 172.76 123.76) (end 173.78 123.76) (width 0.8) (layer "B.Cu") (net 40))
 (segment (start 136.745 96.5) (end 136.745 114.17) (width 0.8) (layer "B.Cu") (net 37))
 (segment (start 163.05 119.0069) (end 163.05 122.736648) (width 0.8) (layer "B.Cu") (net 37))
 (segment (start 137 114.425) (end 158.4681 114.425) (width 0.8) (layer "B.Cu") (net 37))
 (segment (start 171.693352 131.38) (end 173.78 131.38) (width 0.8) (layer "B.Cu") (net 37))
 (segment (start 136.745 114.17) (end 137 114.425) (width 0.8) (layer "B.Cu") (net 37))
 (segment (start 158.4681 114.425) (end 163.05 119.0069) (width 0.8) (layer "B.Cu") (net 37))
 (segment (start 163.05 122.736648) (end 171.693352 131.38) (width 0.8) (layer "B.Cu") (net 37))
 (segment (start 131.665 115.14) (end 134 117.475) (width 0.8) (layer "B.Cu") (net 35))
 (segment (start 131.665 96.5) (end 131.665 115.14) (width 0.8) (layer "B.Cu") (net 35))
 (segment (start 160 124) (end 172.46 136.46) (width 0.8) (layer "B.Cu") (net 35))
 (segment (start 157.204748 117.475) (end 160 120.270252) (width 0.8) (layer "B.Cu") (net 35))
 (segment (start 172.46 136.46) (end 173.78 136.46) (width 0.8) (layer "B.Cu") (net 35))
 (segment (start 160 120.270252) (end 160 124) (width 0.8) (layer "B.Cu") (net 35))
 (segment (start 134 117.475) (end 157.204748 117.475) (width 0.8) (layer "B.Cu") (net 35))
 (segment (start 159.099776 112.9) (end 139.9 112.9) (width 0.8) (layer "B.Cu") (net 38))
 (segment (start 173.78 128.84) (end 171.310028 128.84) (width 0.8) (layer "B.Cu") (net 38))
 (segment (start 139 112) (end 139 99) (width 0.8) (layer "B.Cu") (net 38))
 (segment (start 164.735014 118.535238) (end 159.099776 112.9) (width 0.8) (layer "B.Cu") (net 38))
 (segment (start 164.735014 122.264986) (end 164.735014 118.535238) (width 0.8) (layer "B.Cu") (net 38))
 (segment (start 139.285 98.715) (end 139.285 96.5) (width 0.8) (layer "B.Cu") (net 38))
 (segment (start 171.310028 128.84) (end 164.735014 122.264986) (width 0.8) (layer "B.Cu") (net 38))
 (segment (start 139 99) (end 139.285 98.715) (width 0.8) (layer "B.Cu") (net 38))
 (segment (start 139.9 112.9) (end 139 112) (width 0.8) (layer "B.Cu") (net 38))
 (segment (start 129 116) (end 129.125 115.875) (width 0.8) (layer "B.Cu") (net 34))
 (segment (start 157.975 124.397081) (end 157.975 120.401928) (width 0.8) (layer "B.Cu") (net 34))
 (segment (start 132 119) (end 129 116) (width 0.8) (layer "B.Cu") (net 34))
 (segment (start 156.573072 119) (end 132 119) (width 0.8) (layer "B.Cu") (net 34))
 (segment (start 172.577919 139) (end 157.975 124.397081) (width 0.8) (layer "B.Cu") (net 34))
 (segment (start 129.125 115.875) (end 129.125 96.5) (width 0.8) (layer "B.Cu") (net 34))
 (segment (start 173.78 139) (end 172.577919 139) (width 0.8) (layer "B.Cu") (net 34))
 (segment (start 157.975 120.401928) (end 156.573072 119) (width 0.8) (layer "B.Cu") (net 34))
 (segment (start 161.525 119.638576) (end 157.836424 115.95) (width 0.8) (layer "B.Cu") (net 36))
 (segment (start 134 115) (end 134 100) (width 0.8) (layer "B.Cu") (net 36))
 (segment (start 134.95 115.95) (end 134 115) (width 0.8) (layer "B.Cu") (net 36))
 (segment (start 173.78 133.92) (end 172.076676 133.92) (width 0.8) (layer "B.Cu") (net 36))
 (segment (start 172.076676 133.92) (end 161.525 123.368324) (width 0.8) (layer "B.Cu") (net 36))
 (segment (start 161.525 123.368324) (end 161.525 119.638576) (width 0.8) (layer "B.Cu") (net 36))
 (segment (start 134 100) (end 134.205 99.795) (width 0.8) (layer "B.Cu") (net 36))
 (segment (start 134.205 99.795) (end 134.205 96.5) (width 0.8) (layer "B.Cu") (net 36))
 (segment (start 157.836424 115.95) (end 134.95 115.95) (width 0.8) (layer "B.Cu") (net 36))
 (segment (start 173.78 121.22) (end 173.78 120.017919) (width 0.8) (layer "B.Cu") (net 41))
 (segment (start 173.78 120.017919) (end 162.087081 108.325) (width 0.8) (layer "B.Cu") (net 41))
 (segment (start 162.087081 108.325) (end 147.325 108.325) (width 0.8) (layer "B.Cu") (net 41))
 (segment (start 146.905 107.905) (end 146.905 96.5) (width 0.8) (layer "B.Cu") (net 41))
 (segment (start 147.325 108.325) (end 146.905 107.905) (width 0.8) (layer "B.Cu") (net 41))
 (segment (start 130 87.5) (end 120 87.5) (width 0.8) (layer "F.Cu") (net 13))
 (segment (start 129.5 131) (end 120 131) (width 0.8) (layer "F.Cu") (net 13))
 (via (at 120 131) (size 1.5) (drill 0.75) (layers "F.Cu" "B.Cu") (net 13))
 (via (at 129.5 131) (size 1.5) (drill 0.75) (layers "F.Cu" "B.Cu") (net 13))
 (via (at 120 87.5) (size 1.5) (drill 0.75) (layers "F.Cu" "B.Cu") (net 13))
 (via (at 130 87.5) (size 1.5) (drill 0.75) (layers "F.Cu" "B.Cu") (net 13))
 (segment (start 153.68 85.08) (end 132.763324 85.08) (width 0.8) (layer "B.Cu") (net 13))
 (segment (start 132.763324 85.08) (end 132.42 85.08) (width 0.8) (layer "B.Cu") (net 13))
 (segment (start 120 131) (end 120 87.5) (width 0.8) (layer "B.Cu") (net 13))
 (segment (start 129.88 131.38) (end 129.5 131) (width 0.8) (layer "B.Cu") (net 13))
 (segment (start 153.46 131.38) (end 129.88 131.38) (width 0.8) (layer "B.Cu") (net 13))
 (segment (start 132.42 85.08) (end 130 87.5) (width 0.8) (layer "B.Cu") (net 13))
 (segment (start 149 106) (end 149 121) (width 0.8) (layer "F.Cu") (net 9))
 (via (at 149 106) (size 1.5) (drill 0.75) (layers "F.Cu" "B.Cu") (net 9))
 (via (at 149 106) (size 1.5) (drill 0.75) (layers "F.Cu" "B.Cu") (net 9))
 (via (at 149 121) (size 1.5) (drill 0.75) (layers "F.Cu" "B.Cu") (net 9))
 (segment (start 158.195 94.805) (end 151.5 101.5) (width 0.8) (layer "B.Cu") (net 9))
 (segment (start 149 104) (end 149 106) (width 0.8) (layer "B.Cu") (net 9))
 (segment (start 154.897919 72.5) (end 157 72.5) (width 0.8) (layer "B.Cu") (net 9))
 (segment (start 153.68 73.717919) (end 154.897919 72.5) (width 0.8) (layer "B.Cu") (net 9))
 (segment (start 149.22 121.22) (end 149 121) (width 0.8) (layer "B.Cu") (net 9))
 (segment (start 153.46 121.22) (end 149.22 121.22) (width 0.8) (layer "B.Cu") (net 9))
 (segment (start 158.195 73.695) (end 158.195 94.805) (width 0.8) (layer "B.Cu") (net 9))
 (segment (start 157 72.5) (end 158.195 73.695) (width 0.8) (layer "B.Cu") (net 9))
 (segment (start 153.68 74.92) (end 153.68 73.717919) (width 0.8) (layer "B.Cu") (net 9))
 (segment (start 151.5 101.5) (end 149 104) (width 0.8) (layer "B.Cu") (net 9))
 (segment (start 129.5 134) (end 122 134) (width 0.8) (layer "F.Cu") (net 14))
 (segment (start 130 90) (end 122 90) (width 0.8) (layer "F.Cu") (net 14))
 (via (at 122 90) (size 1.5) (drill 0.75) (layers "F.Cu" "B.Cu") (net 14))
 (via (at 122 134) (size 1.5) (drill 0.75) (layers "F.Cu" "B.Cu") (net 14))
 (via (at 129.5 134) (size 1.5) (drill 0.75) (layers "F.Cu" "B.Cu") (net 14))
 (via (at 130 90) (size 1.5) (drill 0.75) (layers "F.Cu" "B.Cu") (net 14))
 (segment (start 122 90) (end 122 134) (width 0.8) (layer "B.Cu") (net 14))
 (segment (start 135.08 133.92) (end 135 134) (width 0.8) (layer "B.Cu") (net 14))
 (segment (start 152.296928 87.62) (end 149.916928 90) (width 0.8) (layer "B.Cu") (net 14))
 (segment (start 135.08 133.92) (end 129.58 133.92) (width 0.8) (layer "B.Cu") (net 14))
 (segment (start 153.68 87.62) (end 152.296928 87.62) (width 0.8) (layer "B.Cu") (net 14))
 (segment (start 129.58 133.92) (end 129.5 134) (width 0.8) (layer "B.Cu") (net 14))
 (segment (start 149.916928 90) (end 130 90) (width 0.8) (layer "B.Cu") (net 14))
 (segment (start 153.46 133.92) (end 135.08 133.92) (width 0.8) (layer "B.Cu") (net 14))
 (segment (start 136.29 66.5) (end 142.149518 66.5) (width 0.8) (layer "B.Cu") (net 10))
 (segment (start 153.46 123.76) (end 127.41 123.76) (width 0.8) (layer "B.Cu") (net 10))
 (segment (start 142.149518 66.5) (end 144.5 68.850482) (width 0.8) (layer "B.Cu") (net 10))
 (segment (start 123.4725 161.021283) (end 123.4725 154.263717) (width 0.8) (layer "B.Cu") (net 10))
 (segment (start 134.19 68.6) (end 134.19 69) (width 0.8) (layer "B.Cu") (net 10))
 (segment (start 136.46 77.46) (end 144.5 77.46) (width 0.8) (layer "B.Cu") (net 10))
 (segment (start 127.15 118.15) (end 127.15 86.77) (width 0.8) (layer "B.Cu") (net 10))
 (segment (start 144.5 68.850482) (end 144.5 77.46) (width 0.8) (layer "B.Cu") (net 10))
 (segment (start 127.15 123.5) (end 127.15 118.15) (width 0.8) (layer "B.Cu") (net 10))
 (segment (start 153.68 77.46) (end 156.473072 77.46) (width 0.8) (layer "B.Cu") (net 10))
 (segment (start 123.4725 154.263717) (end 131.987868 145.748349) (width 0.8) (layer "B.Cu") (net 10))
 (segment (start 136.29 66.5) (end 134.19 68.6) (width 0.8) (layer "B.Cu") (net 10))
 (segment (start 156 123.76) (end 153.46 123.76) (width 0.8) (layer "B.Cu") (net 10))
 (segment (start 125.173717 162.7225) (end 123.4725 161.021283) (width 0.8) (layer "B.Cu") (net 10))
 (segment (start 127.41 123.76) (end 127.15 123.5) (width 0.8) (layer "B.Cu") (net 10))
 (segment (start 125.4975 162.7225) (end 125.173717 162.7225) (width 0.8) (layer "B.Cu") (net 10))
 (segment (start 144.5 77.46) (end 153.68 77.46) (width 0.8) (layer "B.Cu") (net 10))
 (segment (start 127.15 86.77) (end 136.46 77.46) (width 0.8) (layer "B.Cu") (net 10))
 (segment (start 131.987868 141.836217) (end 127.15 136.998349) (width 0.8) (layer "B.Cu") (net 10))
 (segment (start 127.15 136.998349) (end 127.15 123.5) (width 0.8) (layer "B.Cu") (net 10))
 (segment (start 131.987868 145.748349) (end 131.987868 141.836217) (width 0.8) (layer "B.Cu") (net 10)))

